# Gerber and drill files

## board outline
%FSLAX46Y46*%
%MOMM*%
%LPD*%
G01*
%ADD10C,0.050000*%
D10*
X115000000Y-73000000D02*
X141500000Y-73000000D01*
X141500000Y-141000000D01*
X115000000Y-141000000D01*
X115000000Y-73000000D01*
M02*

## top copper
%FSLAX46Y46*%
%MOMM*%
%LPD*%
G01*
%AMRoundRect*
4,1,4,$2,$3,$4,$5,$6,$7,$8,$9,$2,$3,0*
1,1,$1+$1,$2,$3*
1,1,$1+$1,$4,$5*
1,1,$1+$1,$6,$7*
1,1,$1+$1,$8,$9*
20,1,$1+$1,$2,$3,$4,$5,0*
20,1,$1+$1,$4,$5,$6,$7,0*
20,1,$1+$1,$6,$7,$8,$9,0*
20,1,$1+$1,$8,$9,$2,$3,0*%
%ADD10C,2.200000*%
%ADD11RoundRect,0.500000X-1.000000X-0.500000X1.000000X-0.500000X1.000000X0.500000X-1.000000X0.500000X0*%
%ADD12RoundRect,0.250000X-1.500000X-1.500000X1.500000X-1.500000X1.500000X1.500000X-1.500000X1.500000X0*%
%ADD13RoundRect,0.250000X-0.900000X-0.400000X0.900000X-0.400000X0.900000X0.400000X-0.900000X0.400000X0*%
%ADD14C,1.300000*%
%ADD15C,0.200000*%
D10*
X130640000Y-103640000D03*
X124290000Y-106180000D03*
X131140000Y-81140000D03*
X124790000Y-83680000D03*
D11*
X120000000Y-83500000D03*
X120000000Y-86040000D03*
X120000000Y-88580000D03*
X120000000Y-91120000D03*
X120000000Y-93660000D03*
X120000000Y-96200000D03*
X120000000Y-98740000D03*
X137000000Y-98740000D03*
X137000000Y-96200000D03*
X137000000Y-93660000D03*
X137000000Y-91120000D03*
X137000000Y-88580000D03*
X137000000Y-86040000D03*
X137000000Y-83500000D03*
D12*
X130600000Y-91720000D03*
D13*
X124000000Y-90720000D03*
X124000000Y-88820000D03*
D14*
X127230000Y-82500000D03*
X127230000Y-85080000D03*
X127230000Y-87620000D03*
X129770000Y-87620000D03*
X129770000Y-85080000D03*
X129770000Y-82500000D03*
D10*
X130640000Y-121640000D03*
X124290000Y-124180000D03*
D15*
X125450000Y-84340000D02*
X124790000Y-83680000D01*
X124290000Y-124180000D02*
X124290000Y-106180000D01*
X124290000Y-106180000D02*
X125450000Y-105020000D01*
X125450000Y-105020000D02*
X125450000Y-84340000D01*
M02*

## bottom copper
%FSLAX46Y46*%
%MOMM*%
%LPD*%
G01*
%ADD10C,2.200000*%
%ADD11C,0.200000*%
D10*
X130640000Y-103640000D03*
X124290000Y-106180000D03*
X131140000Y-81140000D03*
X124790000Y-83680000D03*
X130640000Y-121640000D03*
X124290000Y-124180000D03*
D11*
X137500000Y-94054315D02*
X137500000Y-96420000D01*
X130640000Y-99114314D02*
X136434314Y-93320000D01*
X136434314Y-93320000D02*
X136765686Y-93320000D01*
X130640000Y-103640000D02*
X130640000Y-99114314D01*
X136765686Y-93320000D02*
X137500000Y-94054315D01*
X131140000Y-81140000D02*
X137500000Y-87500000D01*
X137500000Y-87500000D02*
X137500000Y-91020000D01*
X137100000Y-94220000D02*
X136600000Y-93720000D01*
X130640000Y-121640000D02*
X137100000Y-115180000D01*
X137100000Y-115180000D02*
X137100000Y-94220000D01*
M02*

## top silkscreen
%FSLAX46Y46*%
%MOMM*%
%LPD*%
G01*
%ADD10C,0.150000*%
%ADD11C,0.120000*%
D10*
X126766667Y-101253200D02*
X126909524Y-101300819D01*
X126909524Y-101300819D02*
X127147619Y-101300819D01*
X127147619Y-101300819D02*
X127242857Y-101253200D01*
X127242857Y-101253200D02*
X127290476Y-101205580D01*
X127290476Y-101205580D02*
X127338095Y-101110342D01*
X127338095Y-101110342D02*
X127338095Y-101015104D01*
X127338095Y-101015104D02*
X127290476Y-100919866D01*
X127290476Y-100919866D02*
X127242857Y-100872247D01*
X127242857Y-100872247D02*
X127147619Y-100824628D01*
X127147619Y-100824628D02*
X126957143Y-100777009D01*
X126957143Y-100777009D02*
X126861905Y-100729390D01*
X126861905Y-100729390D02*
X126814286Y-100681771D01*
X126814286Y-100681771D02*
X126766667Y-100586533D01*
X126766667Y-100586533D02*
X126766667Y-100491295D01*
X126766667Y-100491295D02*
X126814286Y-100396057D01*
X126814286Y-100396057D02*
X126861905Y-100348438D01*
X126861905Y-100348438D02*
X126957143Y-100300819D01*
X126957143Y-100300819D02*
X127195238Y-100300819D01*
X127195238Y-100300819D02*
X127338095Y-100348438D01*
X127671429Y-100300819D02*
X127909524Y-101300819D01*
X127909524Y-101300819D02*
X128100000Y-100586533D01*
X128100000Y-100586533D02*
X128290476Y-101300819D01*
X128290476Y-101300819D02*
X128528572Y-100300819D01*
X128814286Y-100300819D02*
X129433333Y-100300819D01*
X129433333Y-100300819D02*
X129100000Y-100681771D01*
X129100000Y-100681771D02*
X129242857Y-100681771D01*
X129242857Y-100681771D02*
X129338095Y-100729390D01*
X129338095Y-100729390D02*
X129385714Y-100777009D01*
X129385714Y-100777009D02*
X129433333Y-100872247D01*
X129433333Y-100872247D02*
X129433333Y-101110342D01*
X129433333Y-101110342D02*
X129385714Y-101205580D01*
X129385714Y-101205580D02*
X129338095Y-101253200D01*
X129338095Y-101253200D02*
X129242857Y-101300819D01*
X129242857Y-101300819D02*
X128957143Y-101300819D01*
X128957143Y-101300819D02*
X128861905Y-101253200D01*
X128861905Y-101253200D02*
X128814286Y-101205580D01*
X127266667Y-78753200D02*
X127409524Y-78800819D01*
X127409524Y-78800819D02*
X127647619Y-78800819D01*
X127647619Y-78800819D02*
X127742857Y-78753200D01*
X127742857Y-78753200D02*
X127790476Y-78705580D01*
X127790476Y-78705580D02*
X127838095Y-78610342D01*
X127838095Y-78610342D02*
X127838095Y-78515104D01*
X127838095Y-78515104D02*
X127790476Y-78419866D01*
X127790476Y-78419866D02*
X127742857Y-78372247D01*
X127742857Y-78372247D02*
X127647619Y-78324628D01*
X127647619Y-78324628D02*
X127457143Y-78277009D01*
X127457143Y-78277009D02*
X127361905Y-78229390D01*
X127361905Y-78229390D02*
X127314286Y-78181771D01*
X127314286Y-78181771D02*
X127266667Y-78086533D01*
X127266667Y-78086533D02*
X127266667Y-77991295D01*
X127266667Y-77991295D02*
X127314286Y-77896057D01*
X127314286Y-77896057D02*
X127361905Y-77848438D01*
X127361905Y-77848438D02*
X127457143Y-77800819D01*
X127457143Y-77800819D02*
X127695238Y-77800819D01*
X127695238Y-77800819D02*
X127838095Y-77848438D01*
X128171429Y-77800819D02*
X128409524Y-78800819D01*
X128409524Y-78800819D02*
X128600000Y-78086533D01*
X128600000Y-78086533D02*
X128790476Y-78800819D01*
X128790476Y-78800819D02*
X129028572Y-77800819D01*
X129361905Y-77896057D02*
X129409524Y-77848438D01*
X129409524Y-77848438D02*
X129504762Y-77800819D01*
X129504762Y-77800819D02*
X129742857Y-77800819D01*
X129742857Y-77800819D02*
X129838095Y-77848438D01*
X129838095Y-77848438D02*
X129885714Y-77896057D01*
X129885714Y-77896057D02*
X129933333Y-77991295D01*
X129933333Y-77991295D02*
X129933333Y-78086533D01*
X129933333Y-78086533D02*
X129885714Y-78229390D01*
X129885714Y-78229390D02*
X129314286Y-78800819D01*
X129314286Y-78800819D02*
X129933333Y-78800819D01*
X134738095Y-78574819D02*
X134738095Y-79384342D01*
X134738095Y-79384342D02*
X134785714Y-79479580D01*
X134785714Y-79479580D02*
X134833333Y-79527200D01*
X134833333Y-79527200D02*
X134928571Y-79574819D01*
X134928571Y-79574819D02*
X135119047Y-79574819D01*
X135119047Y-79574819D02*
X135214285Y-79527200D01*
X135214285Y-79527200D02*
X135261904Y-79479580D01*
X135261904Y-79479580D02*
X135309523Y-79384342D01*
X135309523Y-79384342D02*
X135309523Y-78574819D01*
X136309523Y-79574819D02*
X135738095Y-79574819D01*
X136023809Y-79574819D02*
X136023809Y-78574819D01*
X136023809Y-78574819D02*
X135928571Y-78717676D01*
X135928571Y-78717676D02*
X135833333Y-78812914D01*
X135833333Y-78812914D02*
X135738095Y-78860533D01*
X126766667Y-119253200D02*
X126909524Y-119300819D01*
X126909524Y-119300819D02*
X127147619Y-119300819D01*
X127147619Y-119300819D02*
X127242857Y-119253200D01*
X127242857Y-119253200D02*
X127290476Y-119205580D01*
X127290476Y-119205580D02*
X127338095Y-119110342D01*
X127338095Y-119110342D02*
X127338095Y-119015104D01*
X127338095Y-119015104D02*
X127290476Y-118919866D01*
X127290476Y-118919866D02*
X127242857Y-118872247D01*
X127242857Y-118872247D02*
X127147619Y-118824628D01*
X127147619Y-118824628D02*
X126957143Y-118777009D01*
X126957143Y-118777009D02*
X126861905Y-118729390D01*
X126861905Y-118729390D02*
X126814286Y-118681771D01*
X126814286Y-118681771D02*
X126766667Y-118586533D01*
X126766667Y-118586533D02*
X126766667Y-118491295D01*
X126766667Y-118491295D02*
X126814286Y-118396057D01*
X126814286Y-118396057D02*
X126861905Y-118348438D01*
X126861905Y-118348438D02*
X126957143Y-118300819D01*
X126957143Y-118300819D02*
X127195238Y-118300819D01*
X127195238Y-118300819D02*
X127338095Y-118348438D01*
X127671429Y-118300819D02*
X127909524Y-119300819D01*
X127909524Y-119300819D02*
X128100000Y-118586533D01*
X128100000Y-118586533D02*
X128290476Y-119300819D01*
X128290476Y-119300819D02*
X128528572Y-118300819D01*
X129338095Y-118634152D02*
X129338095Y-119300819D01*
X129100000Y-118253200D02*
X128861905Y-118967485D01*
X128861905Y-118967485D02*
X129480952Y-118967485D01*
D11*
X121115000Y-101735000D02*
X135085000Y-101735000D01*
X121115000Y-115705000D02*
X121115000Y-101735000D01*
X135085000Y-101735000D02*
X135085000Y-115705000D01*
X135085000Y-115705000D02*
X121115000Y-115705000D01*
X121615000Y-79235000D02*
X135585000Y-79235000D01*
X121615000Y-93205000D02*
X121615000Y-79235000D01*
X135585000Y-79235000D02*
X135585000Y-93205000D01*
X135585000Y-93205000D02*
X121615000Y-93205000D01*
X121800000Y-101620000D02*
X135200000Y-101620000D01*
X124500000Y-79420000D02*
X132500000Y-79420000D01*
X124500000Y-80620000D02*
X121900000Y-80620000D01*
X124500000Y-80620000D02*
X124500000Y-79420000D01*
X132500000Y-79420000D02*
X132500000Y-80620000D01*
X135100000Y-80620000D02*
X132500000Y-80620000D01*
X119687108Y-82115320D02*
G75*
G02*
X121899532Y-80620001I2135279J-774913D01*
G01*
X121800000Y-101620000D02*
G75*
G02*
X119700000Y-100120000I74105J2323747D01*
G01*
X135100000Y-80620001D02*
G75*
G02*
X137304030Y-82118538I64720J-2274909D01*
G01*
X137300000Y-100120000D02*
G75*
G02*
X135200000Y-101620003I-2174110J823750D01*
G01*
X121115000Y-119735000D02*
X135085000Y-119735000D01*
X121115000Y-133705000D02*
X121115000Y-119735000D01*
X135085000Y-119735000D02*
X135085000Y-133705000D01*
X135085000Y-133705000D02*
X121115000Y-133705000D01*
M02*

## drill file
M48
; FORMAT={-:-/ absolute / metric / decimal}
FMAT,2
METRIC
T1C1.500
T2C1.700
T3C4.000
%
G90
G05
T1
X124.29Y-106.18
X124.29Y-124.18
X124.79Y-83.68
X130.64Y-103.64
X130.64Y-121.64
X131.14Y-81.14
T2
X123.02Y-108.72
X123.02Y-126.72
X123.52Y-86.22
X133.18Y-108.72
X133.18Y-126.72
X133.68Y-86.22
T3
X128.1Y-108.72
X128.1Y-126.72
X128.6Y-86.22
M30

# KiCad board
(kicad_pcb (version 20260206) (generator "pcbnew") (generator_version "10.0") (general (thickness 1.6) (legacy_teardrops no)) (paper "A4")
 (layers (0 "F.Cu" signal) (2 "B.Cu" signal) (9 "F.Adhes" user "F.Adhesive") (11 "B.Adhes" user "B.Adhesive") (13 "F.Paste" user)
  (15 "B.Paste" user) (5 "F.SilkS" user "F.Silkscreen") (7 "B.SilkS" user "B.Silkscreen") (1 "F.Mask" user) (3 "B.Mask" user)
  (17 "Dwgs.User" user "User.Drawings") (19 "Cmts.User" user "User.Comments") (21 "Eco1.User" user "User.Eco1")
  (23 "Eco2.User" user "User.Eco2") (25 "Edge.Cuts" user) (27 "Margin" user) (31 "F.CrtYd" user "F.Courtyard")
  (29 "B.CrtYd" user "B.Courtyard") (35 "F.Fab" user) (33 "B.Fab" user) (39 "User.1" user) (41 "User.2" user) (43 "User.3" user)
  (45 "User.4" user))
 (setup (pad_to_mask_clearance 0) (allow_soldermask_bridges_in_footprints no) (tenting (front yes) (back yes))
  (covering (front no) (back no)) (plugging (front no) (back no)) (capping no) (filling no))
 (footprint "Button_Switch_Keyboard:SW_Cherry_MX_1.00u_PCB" (layer "F.Cu") (at 130.64 103.64)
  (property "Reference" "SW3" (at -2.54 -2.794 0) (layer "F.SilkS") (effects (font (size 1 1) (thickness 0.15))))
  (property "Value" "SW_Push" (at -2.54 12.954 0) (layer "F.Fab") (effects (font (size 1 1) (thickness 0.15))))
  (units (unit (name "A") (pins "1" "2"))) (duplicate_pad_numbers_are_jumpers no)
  (fp_line (start -9.525 -1.905) (end 4.445 -1.905) (stroke (width 0.12) (type solid)) (layer "F.SilkS"))
  (fp_line (start -9.525 12.065) (end -9.525 -1.905) (stroke (width 0.12) (type solid)) (layer "F.SilkS"))
  (fp_line (start 4.445 -1.905) (end 4.445 12.065) (stroke (width 0.12) (type solid)) (layer "F.SilkS"))
  (fp_line (start 4.445 12.065) (end -9.525 12.065) (stroke (width 0.12) (type solid)) (layer "F.SilkS"))
  (pad "" np_thru_hole circle (at -7.62 5.08) (size 1.7 1.7) (drill 1.7) (layers "*.Cu" "*.Mask"))
  (pad "" np_thru_hole circle (at -2.54 5.08) (size 4 4) (drill 4) (layers "*.Cu" "*.Mask"))
  (pad "" np_thru_hole circle (at 2.54 5.08) (size 1.7 1.7) (drill 1.7) (layers "*.Cu" "*.Mask"))
  (pad "1" thru_hole circle (at 0 0) (size 2.2 2.2) (drill 1.5) (layers "*.Cu" "*.Mask") (remove_unused_layers no)
   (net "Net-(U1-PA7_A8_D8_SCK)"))
  (pad "2" thru_hole circle (at -6.35 2.54) (size 2.2 2.2) (drill 1.5) (layers "*.Cu" "*.Mask") (remove_unused_layers no) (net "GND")))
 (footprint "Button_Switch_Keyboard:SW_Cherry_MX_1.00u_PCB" (layer "F.Cu") (at 131.14 81.14)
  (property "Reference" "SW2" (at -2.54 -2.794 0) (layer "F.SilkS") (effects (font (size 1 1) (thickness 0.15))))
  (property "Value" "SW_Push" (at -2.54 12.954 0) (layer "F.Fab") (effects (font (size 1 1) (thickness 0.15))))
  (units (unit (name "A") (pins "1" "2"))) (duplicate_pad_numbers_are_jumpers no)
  (fp_line (start -9.525 -1.905) (end 4.445 -1.905) (stroke (width 0.12) (type solid)) (layer "F.SilkS"))
  (fp_line (start -9.525 12.065) (end -9.525 -1.905) (stroke (width 0.12) (type solid)) (layer "F.SilkS"))
  (fp_line (start 4.445 -1.905) (end 4.445 12.065) (stroke (width 0.12) (type solid)) (layer "F.SilkS"))
  (fp_line (start 4.445 12.065) (end -9.525 12.065) (stroke (width 0.12) (type solid)) (layer "F.SilkS"))
  (pad "" np_thru_hole circle (at -7.62 5.08) (size 1.7 1.7) (drill 1.7) (layers "*.Cu" "*.Mask"))
  (pad "" np_thru_hole circle (at -2.54 5.08) (size 4 4) (drill 4) (layers "*.Cu" "*.Mask"))
  (pad "" np_thru_hole circle (at 2.54 5.08) (size 1.7 1.7) (drill 1.7) (layers "*.Cu" "*.Mask"))
  (pad "1" thru_hole circle (at 0 0) (size 2.2 2.2) (drill 1.5) (layers "*.Cu" "*.Mask") (remove_unused_layers no)
   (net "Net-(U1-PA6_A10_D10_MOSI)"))
  (pad "2" thru_hole circle (at -6.35 2.54) (size 2.2 2.2) (drill 1.5) (layers "*.Cu" "*.Mask") (remove_unused_layers no) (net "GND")))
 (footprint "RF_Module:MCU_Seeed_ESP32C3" (layer "F.Cu") (at 128.5 91.12)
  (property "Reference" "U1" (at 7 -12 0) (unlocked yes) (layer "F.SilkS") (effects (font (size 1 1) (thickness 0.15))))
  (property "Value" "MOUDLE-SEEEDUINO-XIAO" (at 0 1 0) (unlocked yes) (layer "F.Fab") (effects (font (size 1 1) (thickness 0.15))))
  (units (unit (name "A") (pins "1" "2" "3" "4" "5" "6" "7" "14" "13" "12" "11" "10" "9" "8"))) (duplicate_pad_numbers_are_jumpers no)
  (fp_line (start -6.7 10.5) (end 6.7 10.5) (stroke (width 0.12) (type default)) (layer "F.SilkS"))
  (fp_line (start -4 -11.7) (end 4 -11.7) (stroke (width 0.12) (type default)) (layer "F.SilkS"))
  (fp_line (start -4 -10.5) (end -6.6 -10.5) (stroke (width 0.12) (type default)) (layer "F.SilkS"))
  (fp_line (start -4 -10.5) (end -4 -11.7) (stroke (width 0.12) (type default)) (layer "F.SilkS"))
  (fp_line (start 4 -11.7) (end 4 -10.5) (stroke (width 0.12) (type default)) (layer "F.SilkS"))
  (fp_line (start 6.6 -10.5) (end 4 -10.5) (stroke (width 0.12) (type default)) (layer "F.SilkS"))
  (fp_arc (start -8.812892 -9.00468) (mid -7.949609 -10.111769) (end -6.600468 -10.499999) (stroke (width 0.12) (type default))
   (layer "F.SilkS"))
  (fp_arc (start -6.7 10.5) (mid -7.977232 10.068125) (end -8.8 9) (stroke (width 0.12) (type default)) (layer "F.SilkS"))
  (fp_arc (start 6.6 -10.499999) (mid 7.944325 -10.107116) (end 8.804034 -9.001464) (stroke (width 0.12) (type default)) (layer "F.SilkS"))
  (fp_arc (start 8.8 9) (mid 7.977232 10.068125) (end 6.7 10.5) (stroke (width 0.12) (type default)) (layer "F.SilkS"))
  (pad "" smd roundrect (at 1.1 -0.4) (size 1.5 1.5) (layers "F.Paste") (roundrect_rratio 0.1666666667))
  (pad "" smd roundrect (at 1.1 1.6) (size 1.5 1.5) (layers "F.Paste") (roundrect_rratio 0.1666666667))
  (pad "" smd roundrect (at 3.1 -0.4) (size 1.5 1.5) (layers "F.Paste") (roundrect_rratio 0.1666666667))
  (pad "" smd roundrect (at 3.1 1.6) (size 1.5 1.5) (layers "F.Paste") (roundrect_rratio 0.1666666667))
  (pad "1" smd roundrect (at -8.5 -7.62) (size 3 2) (layers "F.Cu" "F.Mask" "F.Paste") (roundrect_rratio 0.25)
   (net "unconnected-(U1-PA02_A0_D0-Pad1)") (thermal_bridge_angle 45))
  (pad "2" smd roundrect (at -8.5 -5.08) (size 3 2) (layers "F.Cu" "F.Mask" "F.Paste") (roundrect_rratio 0.25)
   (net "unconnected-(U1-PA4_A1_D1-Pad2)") (thermal_bridge_angle 45))
  (pad "3" smd roundrect (at -8.5 -2.54) (size 3 2) (layers "F.Cu" "F.Mask" "F.Paste") (roundrect_rratio 0.25)
   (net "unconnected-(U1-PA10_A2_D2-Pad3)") (thermal_bridge_angle 45))
  (pad "4" smd roundrect (at -8.5 0) (size 3 2) (layers "F.Cu" "F.Mask" "F.Paste") (roundrect_rratio 0.25)
   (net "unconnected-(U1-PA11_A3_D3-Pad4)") (thermal_bridge_angle 45))
  (pad "5" smd roundrect (at -8.5 2.54) (size 3 2) (layers "F.Cu" "F.Mask" "F.Paste") (roundrect_rratio 0.25)
   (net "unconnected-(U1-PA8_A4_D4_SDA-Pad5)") (thermal_bridge_angle 45))
  (pad "6" smd roundrect (at -8.5 5.08) (size 3 2) (layers "F.Cu" "F.Mask" "F.Paste") (roundrect_rratio 0.25)
   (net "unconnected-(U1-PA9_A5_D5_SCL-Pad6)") (thermal_bridge_angle 45))
  (pad "7" smd roundrect (at -8.5 7.62) (size 3 2) (layers "F.Cu" "F.Mask" "F.Paste") (roundrect_rratio 0.25)
   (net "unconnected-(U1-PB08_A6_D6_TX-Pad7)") (thermal_bridge_angle 45))
  (pad "8" smd roundrect (at 8.5 7.62) (size 3 2) (layers "F.Cu" "F.Mask" "F.Paste") (roundrect_rratio 0.25)
   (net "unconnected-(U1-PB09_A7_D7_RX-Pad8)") (thermal_bridge_angle 45))
  (pad "9" smd roundrect (at 8.5 5.08) (size 3 2) (layers "F.Cu" "F.Mask" "F.Paste") (roundrect_rratio 0.25) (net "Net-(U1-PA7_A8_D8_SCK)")
   (thermal_bridge_angle 45))
  (pad "10" smd roundrect (at 8.5 2.54) (size 3 2) (layers "F.Cu" "F.Mask" "F.Paste") (roundrect_rratio 0.25)
   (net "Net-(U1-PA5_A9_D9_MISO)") (thermal_bridge_angle 45))
  (pad "11" smd roundrect (at 8.5 0) (size 3 2) (layers "F.Cu" "F.Mask" "F.Paste") (roundrect_rratio 0.25) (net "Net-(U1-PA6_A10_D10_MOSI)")
   (thermal_bridge_angle 45))
  (pad "12" smd roundrect (at 8.5 -2.54) (size 3 2) (layers "F.Cu" "F.Mask" "F.Paste") (roundrect_rratio 0.25)
   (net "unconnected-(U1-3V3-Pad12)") (thermal_bridge_angle 45))
  (pad "13" smd roundrect (at 8.5 -5.08) (size 3 2) (layers "F.Cu" "F.Mask" "F.Paste") (roundrect_rratio 0.25) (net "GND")
   (thermal_bridge_angle 45))
  (pad "14" smd roundrect (at 8.5 -7.62) (size 3 2) (layers "F.Cu" "F.Mask" "F.Paste") (roundrect_rratio 0.25)
   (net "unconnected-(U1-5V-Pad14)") (thermal_bridge_angle 45))
  (pad "15" smd roundrect (at 2.1 0.6) (size 3.5 3.5) (layers "F.Cu" "F.Mask") (roundrect_rratio 0.07142857143))
  (pad "16" smd roundrect (at -4.5 -0.4) (size 2.3 1.3) (layers "F.Cu" "F.Mask" "F.Paste") (roundrect_rratio 0.1923076923))
  (pad "17" smd roundrect (at -4.5 -2.3) (size 2.3 1.3) (layers "F.Cu" "F.Mask" "F.Paste") (roundrect_rratio 0.1923076923))
  (pad "18" smd circle (at -1.27 -8.62) (size 1.3 1.3) (layers "F.Cu" "F.Mask" "F.Paste"))
  (pad "19" smd circle (at -1.27 -6.04) (size 1.3 1.3) (layers "F.Cu" "F.Mask" "F.Paste"))
  (pad "20" smd circle (at -1.27 -3.5) (size 1.3 1.3) (layers "F.Cu" "F.Mask" "F.Paste"))
  (pad "21" smd circle (at 1.27 -3.5) (size 1.3 1.3) (layers "F.Cu" "F.Mask" "F.Paste"))
  (pad "22" smd circle (at 1.27 -6.04) (size 1.3 1.3) (layers "F.Cu" "F.Mask" "F.Paste"))
  (pad "23" smd circle (at 1.27 -8.62) (size 1.3 1.3) (layers "F.Cu" "F.Mask" "F.Paste")))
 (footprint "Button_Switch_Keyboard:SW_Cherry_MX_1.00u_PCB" (layer "F.Cu") (at 130.64 121.64)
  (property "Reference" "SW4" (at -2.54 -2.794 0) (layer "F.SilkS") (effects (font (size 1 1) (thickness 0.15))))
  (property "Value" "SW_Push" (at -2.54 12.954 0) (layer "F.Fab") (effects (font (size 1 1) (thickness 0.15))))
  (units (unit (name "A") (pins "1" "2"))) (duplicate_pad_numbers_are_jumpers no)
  (fp_line (start -9.525 -1.905) (end 4.445 -1.905) (stroke (width 0.12) (type solid)) (layer "F.SilkS"))
  (fp_line (start -9.525 12.065) (end -9.525 -1.905) (stroke (width 0.12) (type solid)) (layer "F.SilkS"))
  (fp_line (start 4.445 -1.905) (end 4.445 12.065) (stroke (width 0.12) (type solid)) (layer "F.SilkS"))
  (fp_line (start 4.445 12.065) (end -9.525 12.065) (stroke (width 0.12) (type solid)) (layer "F.SilkS"))
  (pad "" np_thru_hole circle (at -7.62 5.08) (size 1.7 1.7) (drill 1.7) (layers "*.Cu" "*.Mask"))
  (pad "" np_thru_hole circle (at -2.54 5.08) (size 4 4) (drill 4) (layers "*.Cu" "*.Mask"))
  (pad "" np_thru_hole circle (at 2.54 5.08) (size 1.7 1.7) (drill 1.7) (layers "*.Cu" "*.Mask"))
  (pad "1" thru_hole circle (at 0 0) (size 2.2 2.2) (drill 1.5) (layers "*.Cu" "*.Mask") (remove_unused_layers no)
   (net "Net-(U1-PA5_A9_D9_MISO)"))
  (pad "2" thru_hole circle (at -6.35 2.54) (size 2.2 2.2) (drill 1.5) (layers "*.Cu" "*.Mask") (remove_unused_layers no) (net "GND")))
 (gr_rect (start 115 73) (end 141.5 141) (stroke (width 0.05) (type default)) (fill no) (layer "Edge.Cuts"))
 (segment (start 137.5 94.054315) (end 137.5 96.42) (width 0.2) (layer "B.Cu") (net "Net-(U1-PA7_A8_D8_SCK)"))
 (segment (start 130.64 99.114314) (end 136.434314 93.32) (width 0.2) (layer "B.Cu") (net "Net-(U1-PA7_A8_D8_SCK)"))
 (segment (start 136.434314 93.32) (end 136.765686 93.32) (width 0.2) (layer "B.Cu") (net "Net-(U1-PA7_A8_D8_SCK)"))
 (segment (start 130.64 103.64) (end 130.64 99.114314) (width 0.2) (layer "B.Cu") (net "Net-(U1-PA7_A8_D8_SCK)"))
 (segment (start 136.765686 93.32) (end 137.5 94.054315) (width 0.2) (layer "B.Cu") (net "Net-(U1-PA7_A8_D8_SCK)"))
 (segment (start 125.45 84.34) (end 124.79 83.68) (width 0.2) (layer "F.Cu") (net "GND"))
 (segment (start 124.29 124.18) (end 124.29 106.18) (width 0.2) (layer "F.Cu") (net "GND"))
 (segment (start 124.29 106.18) (end 125.45 105.02) (width 0.2) (layer "F.Cu") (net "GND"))
 (segment (start 125.45 105.02) (end 125.45 84.34) (width 0.2) (layer "F.Cu") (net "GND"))
 (segment (start 131.14 81.14) (end 137.5 87.5) (width 0.2) (layer "B.Cu") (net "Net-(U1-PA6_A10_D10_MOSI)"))
 (segment (start 137.5 87.5) (end 137.5 91.02) (width 0.2) (layer "B.Cu") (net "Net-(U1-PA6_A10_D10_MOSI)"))
 (segment (start 137.1 94.22) (end 136.6 93.72) (width 0.2) (layer "B.Cu") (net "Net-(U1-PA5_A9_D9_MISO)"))
 (segment (start 130.64 121.64) (end 137.1 115.18) (width 0.2) (layer "B.Cu") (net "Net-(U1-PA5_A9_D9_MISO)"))
 (segment (start 137.1 115.18) (end 137.1 94.22) (width 0.2) (layer "B.Cu") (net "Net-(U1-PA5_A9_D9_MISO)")))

